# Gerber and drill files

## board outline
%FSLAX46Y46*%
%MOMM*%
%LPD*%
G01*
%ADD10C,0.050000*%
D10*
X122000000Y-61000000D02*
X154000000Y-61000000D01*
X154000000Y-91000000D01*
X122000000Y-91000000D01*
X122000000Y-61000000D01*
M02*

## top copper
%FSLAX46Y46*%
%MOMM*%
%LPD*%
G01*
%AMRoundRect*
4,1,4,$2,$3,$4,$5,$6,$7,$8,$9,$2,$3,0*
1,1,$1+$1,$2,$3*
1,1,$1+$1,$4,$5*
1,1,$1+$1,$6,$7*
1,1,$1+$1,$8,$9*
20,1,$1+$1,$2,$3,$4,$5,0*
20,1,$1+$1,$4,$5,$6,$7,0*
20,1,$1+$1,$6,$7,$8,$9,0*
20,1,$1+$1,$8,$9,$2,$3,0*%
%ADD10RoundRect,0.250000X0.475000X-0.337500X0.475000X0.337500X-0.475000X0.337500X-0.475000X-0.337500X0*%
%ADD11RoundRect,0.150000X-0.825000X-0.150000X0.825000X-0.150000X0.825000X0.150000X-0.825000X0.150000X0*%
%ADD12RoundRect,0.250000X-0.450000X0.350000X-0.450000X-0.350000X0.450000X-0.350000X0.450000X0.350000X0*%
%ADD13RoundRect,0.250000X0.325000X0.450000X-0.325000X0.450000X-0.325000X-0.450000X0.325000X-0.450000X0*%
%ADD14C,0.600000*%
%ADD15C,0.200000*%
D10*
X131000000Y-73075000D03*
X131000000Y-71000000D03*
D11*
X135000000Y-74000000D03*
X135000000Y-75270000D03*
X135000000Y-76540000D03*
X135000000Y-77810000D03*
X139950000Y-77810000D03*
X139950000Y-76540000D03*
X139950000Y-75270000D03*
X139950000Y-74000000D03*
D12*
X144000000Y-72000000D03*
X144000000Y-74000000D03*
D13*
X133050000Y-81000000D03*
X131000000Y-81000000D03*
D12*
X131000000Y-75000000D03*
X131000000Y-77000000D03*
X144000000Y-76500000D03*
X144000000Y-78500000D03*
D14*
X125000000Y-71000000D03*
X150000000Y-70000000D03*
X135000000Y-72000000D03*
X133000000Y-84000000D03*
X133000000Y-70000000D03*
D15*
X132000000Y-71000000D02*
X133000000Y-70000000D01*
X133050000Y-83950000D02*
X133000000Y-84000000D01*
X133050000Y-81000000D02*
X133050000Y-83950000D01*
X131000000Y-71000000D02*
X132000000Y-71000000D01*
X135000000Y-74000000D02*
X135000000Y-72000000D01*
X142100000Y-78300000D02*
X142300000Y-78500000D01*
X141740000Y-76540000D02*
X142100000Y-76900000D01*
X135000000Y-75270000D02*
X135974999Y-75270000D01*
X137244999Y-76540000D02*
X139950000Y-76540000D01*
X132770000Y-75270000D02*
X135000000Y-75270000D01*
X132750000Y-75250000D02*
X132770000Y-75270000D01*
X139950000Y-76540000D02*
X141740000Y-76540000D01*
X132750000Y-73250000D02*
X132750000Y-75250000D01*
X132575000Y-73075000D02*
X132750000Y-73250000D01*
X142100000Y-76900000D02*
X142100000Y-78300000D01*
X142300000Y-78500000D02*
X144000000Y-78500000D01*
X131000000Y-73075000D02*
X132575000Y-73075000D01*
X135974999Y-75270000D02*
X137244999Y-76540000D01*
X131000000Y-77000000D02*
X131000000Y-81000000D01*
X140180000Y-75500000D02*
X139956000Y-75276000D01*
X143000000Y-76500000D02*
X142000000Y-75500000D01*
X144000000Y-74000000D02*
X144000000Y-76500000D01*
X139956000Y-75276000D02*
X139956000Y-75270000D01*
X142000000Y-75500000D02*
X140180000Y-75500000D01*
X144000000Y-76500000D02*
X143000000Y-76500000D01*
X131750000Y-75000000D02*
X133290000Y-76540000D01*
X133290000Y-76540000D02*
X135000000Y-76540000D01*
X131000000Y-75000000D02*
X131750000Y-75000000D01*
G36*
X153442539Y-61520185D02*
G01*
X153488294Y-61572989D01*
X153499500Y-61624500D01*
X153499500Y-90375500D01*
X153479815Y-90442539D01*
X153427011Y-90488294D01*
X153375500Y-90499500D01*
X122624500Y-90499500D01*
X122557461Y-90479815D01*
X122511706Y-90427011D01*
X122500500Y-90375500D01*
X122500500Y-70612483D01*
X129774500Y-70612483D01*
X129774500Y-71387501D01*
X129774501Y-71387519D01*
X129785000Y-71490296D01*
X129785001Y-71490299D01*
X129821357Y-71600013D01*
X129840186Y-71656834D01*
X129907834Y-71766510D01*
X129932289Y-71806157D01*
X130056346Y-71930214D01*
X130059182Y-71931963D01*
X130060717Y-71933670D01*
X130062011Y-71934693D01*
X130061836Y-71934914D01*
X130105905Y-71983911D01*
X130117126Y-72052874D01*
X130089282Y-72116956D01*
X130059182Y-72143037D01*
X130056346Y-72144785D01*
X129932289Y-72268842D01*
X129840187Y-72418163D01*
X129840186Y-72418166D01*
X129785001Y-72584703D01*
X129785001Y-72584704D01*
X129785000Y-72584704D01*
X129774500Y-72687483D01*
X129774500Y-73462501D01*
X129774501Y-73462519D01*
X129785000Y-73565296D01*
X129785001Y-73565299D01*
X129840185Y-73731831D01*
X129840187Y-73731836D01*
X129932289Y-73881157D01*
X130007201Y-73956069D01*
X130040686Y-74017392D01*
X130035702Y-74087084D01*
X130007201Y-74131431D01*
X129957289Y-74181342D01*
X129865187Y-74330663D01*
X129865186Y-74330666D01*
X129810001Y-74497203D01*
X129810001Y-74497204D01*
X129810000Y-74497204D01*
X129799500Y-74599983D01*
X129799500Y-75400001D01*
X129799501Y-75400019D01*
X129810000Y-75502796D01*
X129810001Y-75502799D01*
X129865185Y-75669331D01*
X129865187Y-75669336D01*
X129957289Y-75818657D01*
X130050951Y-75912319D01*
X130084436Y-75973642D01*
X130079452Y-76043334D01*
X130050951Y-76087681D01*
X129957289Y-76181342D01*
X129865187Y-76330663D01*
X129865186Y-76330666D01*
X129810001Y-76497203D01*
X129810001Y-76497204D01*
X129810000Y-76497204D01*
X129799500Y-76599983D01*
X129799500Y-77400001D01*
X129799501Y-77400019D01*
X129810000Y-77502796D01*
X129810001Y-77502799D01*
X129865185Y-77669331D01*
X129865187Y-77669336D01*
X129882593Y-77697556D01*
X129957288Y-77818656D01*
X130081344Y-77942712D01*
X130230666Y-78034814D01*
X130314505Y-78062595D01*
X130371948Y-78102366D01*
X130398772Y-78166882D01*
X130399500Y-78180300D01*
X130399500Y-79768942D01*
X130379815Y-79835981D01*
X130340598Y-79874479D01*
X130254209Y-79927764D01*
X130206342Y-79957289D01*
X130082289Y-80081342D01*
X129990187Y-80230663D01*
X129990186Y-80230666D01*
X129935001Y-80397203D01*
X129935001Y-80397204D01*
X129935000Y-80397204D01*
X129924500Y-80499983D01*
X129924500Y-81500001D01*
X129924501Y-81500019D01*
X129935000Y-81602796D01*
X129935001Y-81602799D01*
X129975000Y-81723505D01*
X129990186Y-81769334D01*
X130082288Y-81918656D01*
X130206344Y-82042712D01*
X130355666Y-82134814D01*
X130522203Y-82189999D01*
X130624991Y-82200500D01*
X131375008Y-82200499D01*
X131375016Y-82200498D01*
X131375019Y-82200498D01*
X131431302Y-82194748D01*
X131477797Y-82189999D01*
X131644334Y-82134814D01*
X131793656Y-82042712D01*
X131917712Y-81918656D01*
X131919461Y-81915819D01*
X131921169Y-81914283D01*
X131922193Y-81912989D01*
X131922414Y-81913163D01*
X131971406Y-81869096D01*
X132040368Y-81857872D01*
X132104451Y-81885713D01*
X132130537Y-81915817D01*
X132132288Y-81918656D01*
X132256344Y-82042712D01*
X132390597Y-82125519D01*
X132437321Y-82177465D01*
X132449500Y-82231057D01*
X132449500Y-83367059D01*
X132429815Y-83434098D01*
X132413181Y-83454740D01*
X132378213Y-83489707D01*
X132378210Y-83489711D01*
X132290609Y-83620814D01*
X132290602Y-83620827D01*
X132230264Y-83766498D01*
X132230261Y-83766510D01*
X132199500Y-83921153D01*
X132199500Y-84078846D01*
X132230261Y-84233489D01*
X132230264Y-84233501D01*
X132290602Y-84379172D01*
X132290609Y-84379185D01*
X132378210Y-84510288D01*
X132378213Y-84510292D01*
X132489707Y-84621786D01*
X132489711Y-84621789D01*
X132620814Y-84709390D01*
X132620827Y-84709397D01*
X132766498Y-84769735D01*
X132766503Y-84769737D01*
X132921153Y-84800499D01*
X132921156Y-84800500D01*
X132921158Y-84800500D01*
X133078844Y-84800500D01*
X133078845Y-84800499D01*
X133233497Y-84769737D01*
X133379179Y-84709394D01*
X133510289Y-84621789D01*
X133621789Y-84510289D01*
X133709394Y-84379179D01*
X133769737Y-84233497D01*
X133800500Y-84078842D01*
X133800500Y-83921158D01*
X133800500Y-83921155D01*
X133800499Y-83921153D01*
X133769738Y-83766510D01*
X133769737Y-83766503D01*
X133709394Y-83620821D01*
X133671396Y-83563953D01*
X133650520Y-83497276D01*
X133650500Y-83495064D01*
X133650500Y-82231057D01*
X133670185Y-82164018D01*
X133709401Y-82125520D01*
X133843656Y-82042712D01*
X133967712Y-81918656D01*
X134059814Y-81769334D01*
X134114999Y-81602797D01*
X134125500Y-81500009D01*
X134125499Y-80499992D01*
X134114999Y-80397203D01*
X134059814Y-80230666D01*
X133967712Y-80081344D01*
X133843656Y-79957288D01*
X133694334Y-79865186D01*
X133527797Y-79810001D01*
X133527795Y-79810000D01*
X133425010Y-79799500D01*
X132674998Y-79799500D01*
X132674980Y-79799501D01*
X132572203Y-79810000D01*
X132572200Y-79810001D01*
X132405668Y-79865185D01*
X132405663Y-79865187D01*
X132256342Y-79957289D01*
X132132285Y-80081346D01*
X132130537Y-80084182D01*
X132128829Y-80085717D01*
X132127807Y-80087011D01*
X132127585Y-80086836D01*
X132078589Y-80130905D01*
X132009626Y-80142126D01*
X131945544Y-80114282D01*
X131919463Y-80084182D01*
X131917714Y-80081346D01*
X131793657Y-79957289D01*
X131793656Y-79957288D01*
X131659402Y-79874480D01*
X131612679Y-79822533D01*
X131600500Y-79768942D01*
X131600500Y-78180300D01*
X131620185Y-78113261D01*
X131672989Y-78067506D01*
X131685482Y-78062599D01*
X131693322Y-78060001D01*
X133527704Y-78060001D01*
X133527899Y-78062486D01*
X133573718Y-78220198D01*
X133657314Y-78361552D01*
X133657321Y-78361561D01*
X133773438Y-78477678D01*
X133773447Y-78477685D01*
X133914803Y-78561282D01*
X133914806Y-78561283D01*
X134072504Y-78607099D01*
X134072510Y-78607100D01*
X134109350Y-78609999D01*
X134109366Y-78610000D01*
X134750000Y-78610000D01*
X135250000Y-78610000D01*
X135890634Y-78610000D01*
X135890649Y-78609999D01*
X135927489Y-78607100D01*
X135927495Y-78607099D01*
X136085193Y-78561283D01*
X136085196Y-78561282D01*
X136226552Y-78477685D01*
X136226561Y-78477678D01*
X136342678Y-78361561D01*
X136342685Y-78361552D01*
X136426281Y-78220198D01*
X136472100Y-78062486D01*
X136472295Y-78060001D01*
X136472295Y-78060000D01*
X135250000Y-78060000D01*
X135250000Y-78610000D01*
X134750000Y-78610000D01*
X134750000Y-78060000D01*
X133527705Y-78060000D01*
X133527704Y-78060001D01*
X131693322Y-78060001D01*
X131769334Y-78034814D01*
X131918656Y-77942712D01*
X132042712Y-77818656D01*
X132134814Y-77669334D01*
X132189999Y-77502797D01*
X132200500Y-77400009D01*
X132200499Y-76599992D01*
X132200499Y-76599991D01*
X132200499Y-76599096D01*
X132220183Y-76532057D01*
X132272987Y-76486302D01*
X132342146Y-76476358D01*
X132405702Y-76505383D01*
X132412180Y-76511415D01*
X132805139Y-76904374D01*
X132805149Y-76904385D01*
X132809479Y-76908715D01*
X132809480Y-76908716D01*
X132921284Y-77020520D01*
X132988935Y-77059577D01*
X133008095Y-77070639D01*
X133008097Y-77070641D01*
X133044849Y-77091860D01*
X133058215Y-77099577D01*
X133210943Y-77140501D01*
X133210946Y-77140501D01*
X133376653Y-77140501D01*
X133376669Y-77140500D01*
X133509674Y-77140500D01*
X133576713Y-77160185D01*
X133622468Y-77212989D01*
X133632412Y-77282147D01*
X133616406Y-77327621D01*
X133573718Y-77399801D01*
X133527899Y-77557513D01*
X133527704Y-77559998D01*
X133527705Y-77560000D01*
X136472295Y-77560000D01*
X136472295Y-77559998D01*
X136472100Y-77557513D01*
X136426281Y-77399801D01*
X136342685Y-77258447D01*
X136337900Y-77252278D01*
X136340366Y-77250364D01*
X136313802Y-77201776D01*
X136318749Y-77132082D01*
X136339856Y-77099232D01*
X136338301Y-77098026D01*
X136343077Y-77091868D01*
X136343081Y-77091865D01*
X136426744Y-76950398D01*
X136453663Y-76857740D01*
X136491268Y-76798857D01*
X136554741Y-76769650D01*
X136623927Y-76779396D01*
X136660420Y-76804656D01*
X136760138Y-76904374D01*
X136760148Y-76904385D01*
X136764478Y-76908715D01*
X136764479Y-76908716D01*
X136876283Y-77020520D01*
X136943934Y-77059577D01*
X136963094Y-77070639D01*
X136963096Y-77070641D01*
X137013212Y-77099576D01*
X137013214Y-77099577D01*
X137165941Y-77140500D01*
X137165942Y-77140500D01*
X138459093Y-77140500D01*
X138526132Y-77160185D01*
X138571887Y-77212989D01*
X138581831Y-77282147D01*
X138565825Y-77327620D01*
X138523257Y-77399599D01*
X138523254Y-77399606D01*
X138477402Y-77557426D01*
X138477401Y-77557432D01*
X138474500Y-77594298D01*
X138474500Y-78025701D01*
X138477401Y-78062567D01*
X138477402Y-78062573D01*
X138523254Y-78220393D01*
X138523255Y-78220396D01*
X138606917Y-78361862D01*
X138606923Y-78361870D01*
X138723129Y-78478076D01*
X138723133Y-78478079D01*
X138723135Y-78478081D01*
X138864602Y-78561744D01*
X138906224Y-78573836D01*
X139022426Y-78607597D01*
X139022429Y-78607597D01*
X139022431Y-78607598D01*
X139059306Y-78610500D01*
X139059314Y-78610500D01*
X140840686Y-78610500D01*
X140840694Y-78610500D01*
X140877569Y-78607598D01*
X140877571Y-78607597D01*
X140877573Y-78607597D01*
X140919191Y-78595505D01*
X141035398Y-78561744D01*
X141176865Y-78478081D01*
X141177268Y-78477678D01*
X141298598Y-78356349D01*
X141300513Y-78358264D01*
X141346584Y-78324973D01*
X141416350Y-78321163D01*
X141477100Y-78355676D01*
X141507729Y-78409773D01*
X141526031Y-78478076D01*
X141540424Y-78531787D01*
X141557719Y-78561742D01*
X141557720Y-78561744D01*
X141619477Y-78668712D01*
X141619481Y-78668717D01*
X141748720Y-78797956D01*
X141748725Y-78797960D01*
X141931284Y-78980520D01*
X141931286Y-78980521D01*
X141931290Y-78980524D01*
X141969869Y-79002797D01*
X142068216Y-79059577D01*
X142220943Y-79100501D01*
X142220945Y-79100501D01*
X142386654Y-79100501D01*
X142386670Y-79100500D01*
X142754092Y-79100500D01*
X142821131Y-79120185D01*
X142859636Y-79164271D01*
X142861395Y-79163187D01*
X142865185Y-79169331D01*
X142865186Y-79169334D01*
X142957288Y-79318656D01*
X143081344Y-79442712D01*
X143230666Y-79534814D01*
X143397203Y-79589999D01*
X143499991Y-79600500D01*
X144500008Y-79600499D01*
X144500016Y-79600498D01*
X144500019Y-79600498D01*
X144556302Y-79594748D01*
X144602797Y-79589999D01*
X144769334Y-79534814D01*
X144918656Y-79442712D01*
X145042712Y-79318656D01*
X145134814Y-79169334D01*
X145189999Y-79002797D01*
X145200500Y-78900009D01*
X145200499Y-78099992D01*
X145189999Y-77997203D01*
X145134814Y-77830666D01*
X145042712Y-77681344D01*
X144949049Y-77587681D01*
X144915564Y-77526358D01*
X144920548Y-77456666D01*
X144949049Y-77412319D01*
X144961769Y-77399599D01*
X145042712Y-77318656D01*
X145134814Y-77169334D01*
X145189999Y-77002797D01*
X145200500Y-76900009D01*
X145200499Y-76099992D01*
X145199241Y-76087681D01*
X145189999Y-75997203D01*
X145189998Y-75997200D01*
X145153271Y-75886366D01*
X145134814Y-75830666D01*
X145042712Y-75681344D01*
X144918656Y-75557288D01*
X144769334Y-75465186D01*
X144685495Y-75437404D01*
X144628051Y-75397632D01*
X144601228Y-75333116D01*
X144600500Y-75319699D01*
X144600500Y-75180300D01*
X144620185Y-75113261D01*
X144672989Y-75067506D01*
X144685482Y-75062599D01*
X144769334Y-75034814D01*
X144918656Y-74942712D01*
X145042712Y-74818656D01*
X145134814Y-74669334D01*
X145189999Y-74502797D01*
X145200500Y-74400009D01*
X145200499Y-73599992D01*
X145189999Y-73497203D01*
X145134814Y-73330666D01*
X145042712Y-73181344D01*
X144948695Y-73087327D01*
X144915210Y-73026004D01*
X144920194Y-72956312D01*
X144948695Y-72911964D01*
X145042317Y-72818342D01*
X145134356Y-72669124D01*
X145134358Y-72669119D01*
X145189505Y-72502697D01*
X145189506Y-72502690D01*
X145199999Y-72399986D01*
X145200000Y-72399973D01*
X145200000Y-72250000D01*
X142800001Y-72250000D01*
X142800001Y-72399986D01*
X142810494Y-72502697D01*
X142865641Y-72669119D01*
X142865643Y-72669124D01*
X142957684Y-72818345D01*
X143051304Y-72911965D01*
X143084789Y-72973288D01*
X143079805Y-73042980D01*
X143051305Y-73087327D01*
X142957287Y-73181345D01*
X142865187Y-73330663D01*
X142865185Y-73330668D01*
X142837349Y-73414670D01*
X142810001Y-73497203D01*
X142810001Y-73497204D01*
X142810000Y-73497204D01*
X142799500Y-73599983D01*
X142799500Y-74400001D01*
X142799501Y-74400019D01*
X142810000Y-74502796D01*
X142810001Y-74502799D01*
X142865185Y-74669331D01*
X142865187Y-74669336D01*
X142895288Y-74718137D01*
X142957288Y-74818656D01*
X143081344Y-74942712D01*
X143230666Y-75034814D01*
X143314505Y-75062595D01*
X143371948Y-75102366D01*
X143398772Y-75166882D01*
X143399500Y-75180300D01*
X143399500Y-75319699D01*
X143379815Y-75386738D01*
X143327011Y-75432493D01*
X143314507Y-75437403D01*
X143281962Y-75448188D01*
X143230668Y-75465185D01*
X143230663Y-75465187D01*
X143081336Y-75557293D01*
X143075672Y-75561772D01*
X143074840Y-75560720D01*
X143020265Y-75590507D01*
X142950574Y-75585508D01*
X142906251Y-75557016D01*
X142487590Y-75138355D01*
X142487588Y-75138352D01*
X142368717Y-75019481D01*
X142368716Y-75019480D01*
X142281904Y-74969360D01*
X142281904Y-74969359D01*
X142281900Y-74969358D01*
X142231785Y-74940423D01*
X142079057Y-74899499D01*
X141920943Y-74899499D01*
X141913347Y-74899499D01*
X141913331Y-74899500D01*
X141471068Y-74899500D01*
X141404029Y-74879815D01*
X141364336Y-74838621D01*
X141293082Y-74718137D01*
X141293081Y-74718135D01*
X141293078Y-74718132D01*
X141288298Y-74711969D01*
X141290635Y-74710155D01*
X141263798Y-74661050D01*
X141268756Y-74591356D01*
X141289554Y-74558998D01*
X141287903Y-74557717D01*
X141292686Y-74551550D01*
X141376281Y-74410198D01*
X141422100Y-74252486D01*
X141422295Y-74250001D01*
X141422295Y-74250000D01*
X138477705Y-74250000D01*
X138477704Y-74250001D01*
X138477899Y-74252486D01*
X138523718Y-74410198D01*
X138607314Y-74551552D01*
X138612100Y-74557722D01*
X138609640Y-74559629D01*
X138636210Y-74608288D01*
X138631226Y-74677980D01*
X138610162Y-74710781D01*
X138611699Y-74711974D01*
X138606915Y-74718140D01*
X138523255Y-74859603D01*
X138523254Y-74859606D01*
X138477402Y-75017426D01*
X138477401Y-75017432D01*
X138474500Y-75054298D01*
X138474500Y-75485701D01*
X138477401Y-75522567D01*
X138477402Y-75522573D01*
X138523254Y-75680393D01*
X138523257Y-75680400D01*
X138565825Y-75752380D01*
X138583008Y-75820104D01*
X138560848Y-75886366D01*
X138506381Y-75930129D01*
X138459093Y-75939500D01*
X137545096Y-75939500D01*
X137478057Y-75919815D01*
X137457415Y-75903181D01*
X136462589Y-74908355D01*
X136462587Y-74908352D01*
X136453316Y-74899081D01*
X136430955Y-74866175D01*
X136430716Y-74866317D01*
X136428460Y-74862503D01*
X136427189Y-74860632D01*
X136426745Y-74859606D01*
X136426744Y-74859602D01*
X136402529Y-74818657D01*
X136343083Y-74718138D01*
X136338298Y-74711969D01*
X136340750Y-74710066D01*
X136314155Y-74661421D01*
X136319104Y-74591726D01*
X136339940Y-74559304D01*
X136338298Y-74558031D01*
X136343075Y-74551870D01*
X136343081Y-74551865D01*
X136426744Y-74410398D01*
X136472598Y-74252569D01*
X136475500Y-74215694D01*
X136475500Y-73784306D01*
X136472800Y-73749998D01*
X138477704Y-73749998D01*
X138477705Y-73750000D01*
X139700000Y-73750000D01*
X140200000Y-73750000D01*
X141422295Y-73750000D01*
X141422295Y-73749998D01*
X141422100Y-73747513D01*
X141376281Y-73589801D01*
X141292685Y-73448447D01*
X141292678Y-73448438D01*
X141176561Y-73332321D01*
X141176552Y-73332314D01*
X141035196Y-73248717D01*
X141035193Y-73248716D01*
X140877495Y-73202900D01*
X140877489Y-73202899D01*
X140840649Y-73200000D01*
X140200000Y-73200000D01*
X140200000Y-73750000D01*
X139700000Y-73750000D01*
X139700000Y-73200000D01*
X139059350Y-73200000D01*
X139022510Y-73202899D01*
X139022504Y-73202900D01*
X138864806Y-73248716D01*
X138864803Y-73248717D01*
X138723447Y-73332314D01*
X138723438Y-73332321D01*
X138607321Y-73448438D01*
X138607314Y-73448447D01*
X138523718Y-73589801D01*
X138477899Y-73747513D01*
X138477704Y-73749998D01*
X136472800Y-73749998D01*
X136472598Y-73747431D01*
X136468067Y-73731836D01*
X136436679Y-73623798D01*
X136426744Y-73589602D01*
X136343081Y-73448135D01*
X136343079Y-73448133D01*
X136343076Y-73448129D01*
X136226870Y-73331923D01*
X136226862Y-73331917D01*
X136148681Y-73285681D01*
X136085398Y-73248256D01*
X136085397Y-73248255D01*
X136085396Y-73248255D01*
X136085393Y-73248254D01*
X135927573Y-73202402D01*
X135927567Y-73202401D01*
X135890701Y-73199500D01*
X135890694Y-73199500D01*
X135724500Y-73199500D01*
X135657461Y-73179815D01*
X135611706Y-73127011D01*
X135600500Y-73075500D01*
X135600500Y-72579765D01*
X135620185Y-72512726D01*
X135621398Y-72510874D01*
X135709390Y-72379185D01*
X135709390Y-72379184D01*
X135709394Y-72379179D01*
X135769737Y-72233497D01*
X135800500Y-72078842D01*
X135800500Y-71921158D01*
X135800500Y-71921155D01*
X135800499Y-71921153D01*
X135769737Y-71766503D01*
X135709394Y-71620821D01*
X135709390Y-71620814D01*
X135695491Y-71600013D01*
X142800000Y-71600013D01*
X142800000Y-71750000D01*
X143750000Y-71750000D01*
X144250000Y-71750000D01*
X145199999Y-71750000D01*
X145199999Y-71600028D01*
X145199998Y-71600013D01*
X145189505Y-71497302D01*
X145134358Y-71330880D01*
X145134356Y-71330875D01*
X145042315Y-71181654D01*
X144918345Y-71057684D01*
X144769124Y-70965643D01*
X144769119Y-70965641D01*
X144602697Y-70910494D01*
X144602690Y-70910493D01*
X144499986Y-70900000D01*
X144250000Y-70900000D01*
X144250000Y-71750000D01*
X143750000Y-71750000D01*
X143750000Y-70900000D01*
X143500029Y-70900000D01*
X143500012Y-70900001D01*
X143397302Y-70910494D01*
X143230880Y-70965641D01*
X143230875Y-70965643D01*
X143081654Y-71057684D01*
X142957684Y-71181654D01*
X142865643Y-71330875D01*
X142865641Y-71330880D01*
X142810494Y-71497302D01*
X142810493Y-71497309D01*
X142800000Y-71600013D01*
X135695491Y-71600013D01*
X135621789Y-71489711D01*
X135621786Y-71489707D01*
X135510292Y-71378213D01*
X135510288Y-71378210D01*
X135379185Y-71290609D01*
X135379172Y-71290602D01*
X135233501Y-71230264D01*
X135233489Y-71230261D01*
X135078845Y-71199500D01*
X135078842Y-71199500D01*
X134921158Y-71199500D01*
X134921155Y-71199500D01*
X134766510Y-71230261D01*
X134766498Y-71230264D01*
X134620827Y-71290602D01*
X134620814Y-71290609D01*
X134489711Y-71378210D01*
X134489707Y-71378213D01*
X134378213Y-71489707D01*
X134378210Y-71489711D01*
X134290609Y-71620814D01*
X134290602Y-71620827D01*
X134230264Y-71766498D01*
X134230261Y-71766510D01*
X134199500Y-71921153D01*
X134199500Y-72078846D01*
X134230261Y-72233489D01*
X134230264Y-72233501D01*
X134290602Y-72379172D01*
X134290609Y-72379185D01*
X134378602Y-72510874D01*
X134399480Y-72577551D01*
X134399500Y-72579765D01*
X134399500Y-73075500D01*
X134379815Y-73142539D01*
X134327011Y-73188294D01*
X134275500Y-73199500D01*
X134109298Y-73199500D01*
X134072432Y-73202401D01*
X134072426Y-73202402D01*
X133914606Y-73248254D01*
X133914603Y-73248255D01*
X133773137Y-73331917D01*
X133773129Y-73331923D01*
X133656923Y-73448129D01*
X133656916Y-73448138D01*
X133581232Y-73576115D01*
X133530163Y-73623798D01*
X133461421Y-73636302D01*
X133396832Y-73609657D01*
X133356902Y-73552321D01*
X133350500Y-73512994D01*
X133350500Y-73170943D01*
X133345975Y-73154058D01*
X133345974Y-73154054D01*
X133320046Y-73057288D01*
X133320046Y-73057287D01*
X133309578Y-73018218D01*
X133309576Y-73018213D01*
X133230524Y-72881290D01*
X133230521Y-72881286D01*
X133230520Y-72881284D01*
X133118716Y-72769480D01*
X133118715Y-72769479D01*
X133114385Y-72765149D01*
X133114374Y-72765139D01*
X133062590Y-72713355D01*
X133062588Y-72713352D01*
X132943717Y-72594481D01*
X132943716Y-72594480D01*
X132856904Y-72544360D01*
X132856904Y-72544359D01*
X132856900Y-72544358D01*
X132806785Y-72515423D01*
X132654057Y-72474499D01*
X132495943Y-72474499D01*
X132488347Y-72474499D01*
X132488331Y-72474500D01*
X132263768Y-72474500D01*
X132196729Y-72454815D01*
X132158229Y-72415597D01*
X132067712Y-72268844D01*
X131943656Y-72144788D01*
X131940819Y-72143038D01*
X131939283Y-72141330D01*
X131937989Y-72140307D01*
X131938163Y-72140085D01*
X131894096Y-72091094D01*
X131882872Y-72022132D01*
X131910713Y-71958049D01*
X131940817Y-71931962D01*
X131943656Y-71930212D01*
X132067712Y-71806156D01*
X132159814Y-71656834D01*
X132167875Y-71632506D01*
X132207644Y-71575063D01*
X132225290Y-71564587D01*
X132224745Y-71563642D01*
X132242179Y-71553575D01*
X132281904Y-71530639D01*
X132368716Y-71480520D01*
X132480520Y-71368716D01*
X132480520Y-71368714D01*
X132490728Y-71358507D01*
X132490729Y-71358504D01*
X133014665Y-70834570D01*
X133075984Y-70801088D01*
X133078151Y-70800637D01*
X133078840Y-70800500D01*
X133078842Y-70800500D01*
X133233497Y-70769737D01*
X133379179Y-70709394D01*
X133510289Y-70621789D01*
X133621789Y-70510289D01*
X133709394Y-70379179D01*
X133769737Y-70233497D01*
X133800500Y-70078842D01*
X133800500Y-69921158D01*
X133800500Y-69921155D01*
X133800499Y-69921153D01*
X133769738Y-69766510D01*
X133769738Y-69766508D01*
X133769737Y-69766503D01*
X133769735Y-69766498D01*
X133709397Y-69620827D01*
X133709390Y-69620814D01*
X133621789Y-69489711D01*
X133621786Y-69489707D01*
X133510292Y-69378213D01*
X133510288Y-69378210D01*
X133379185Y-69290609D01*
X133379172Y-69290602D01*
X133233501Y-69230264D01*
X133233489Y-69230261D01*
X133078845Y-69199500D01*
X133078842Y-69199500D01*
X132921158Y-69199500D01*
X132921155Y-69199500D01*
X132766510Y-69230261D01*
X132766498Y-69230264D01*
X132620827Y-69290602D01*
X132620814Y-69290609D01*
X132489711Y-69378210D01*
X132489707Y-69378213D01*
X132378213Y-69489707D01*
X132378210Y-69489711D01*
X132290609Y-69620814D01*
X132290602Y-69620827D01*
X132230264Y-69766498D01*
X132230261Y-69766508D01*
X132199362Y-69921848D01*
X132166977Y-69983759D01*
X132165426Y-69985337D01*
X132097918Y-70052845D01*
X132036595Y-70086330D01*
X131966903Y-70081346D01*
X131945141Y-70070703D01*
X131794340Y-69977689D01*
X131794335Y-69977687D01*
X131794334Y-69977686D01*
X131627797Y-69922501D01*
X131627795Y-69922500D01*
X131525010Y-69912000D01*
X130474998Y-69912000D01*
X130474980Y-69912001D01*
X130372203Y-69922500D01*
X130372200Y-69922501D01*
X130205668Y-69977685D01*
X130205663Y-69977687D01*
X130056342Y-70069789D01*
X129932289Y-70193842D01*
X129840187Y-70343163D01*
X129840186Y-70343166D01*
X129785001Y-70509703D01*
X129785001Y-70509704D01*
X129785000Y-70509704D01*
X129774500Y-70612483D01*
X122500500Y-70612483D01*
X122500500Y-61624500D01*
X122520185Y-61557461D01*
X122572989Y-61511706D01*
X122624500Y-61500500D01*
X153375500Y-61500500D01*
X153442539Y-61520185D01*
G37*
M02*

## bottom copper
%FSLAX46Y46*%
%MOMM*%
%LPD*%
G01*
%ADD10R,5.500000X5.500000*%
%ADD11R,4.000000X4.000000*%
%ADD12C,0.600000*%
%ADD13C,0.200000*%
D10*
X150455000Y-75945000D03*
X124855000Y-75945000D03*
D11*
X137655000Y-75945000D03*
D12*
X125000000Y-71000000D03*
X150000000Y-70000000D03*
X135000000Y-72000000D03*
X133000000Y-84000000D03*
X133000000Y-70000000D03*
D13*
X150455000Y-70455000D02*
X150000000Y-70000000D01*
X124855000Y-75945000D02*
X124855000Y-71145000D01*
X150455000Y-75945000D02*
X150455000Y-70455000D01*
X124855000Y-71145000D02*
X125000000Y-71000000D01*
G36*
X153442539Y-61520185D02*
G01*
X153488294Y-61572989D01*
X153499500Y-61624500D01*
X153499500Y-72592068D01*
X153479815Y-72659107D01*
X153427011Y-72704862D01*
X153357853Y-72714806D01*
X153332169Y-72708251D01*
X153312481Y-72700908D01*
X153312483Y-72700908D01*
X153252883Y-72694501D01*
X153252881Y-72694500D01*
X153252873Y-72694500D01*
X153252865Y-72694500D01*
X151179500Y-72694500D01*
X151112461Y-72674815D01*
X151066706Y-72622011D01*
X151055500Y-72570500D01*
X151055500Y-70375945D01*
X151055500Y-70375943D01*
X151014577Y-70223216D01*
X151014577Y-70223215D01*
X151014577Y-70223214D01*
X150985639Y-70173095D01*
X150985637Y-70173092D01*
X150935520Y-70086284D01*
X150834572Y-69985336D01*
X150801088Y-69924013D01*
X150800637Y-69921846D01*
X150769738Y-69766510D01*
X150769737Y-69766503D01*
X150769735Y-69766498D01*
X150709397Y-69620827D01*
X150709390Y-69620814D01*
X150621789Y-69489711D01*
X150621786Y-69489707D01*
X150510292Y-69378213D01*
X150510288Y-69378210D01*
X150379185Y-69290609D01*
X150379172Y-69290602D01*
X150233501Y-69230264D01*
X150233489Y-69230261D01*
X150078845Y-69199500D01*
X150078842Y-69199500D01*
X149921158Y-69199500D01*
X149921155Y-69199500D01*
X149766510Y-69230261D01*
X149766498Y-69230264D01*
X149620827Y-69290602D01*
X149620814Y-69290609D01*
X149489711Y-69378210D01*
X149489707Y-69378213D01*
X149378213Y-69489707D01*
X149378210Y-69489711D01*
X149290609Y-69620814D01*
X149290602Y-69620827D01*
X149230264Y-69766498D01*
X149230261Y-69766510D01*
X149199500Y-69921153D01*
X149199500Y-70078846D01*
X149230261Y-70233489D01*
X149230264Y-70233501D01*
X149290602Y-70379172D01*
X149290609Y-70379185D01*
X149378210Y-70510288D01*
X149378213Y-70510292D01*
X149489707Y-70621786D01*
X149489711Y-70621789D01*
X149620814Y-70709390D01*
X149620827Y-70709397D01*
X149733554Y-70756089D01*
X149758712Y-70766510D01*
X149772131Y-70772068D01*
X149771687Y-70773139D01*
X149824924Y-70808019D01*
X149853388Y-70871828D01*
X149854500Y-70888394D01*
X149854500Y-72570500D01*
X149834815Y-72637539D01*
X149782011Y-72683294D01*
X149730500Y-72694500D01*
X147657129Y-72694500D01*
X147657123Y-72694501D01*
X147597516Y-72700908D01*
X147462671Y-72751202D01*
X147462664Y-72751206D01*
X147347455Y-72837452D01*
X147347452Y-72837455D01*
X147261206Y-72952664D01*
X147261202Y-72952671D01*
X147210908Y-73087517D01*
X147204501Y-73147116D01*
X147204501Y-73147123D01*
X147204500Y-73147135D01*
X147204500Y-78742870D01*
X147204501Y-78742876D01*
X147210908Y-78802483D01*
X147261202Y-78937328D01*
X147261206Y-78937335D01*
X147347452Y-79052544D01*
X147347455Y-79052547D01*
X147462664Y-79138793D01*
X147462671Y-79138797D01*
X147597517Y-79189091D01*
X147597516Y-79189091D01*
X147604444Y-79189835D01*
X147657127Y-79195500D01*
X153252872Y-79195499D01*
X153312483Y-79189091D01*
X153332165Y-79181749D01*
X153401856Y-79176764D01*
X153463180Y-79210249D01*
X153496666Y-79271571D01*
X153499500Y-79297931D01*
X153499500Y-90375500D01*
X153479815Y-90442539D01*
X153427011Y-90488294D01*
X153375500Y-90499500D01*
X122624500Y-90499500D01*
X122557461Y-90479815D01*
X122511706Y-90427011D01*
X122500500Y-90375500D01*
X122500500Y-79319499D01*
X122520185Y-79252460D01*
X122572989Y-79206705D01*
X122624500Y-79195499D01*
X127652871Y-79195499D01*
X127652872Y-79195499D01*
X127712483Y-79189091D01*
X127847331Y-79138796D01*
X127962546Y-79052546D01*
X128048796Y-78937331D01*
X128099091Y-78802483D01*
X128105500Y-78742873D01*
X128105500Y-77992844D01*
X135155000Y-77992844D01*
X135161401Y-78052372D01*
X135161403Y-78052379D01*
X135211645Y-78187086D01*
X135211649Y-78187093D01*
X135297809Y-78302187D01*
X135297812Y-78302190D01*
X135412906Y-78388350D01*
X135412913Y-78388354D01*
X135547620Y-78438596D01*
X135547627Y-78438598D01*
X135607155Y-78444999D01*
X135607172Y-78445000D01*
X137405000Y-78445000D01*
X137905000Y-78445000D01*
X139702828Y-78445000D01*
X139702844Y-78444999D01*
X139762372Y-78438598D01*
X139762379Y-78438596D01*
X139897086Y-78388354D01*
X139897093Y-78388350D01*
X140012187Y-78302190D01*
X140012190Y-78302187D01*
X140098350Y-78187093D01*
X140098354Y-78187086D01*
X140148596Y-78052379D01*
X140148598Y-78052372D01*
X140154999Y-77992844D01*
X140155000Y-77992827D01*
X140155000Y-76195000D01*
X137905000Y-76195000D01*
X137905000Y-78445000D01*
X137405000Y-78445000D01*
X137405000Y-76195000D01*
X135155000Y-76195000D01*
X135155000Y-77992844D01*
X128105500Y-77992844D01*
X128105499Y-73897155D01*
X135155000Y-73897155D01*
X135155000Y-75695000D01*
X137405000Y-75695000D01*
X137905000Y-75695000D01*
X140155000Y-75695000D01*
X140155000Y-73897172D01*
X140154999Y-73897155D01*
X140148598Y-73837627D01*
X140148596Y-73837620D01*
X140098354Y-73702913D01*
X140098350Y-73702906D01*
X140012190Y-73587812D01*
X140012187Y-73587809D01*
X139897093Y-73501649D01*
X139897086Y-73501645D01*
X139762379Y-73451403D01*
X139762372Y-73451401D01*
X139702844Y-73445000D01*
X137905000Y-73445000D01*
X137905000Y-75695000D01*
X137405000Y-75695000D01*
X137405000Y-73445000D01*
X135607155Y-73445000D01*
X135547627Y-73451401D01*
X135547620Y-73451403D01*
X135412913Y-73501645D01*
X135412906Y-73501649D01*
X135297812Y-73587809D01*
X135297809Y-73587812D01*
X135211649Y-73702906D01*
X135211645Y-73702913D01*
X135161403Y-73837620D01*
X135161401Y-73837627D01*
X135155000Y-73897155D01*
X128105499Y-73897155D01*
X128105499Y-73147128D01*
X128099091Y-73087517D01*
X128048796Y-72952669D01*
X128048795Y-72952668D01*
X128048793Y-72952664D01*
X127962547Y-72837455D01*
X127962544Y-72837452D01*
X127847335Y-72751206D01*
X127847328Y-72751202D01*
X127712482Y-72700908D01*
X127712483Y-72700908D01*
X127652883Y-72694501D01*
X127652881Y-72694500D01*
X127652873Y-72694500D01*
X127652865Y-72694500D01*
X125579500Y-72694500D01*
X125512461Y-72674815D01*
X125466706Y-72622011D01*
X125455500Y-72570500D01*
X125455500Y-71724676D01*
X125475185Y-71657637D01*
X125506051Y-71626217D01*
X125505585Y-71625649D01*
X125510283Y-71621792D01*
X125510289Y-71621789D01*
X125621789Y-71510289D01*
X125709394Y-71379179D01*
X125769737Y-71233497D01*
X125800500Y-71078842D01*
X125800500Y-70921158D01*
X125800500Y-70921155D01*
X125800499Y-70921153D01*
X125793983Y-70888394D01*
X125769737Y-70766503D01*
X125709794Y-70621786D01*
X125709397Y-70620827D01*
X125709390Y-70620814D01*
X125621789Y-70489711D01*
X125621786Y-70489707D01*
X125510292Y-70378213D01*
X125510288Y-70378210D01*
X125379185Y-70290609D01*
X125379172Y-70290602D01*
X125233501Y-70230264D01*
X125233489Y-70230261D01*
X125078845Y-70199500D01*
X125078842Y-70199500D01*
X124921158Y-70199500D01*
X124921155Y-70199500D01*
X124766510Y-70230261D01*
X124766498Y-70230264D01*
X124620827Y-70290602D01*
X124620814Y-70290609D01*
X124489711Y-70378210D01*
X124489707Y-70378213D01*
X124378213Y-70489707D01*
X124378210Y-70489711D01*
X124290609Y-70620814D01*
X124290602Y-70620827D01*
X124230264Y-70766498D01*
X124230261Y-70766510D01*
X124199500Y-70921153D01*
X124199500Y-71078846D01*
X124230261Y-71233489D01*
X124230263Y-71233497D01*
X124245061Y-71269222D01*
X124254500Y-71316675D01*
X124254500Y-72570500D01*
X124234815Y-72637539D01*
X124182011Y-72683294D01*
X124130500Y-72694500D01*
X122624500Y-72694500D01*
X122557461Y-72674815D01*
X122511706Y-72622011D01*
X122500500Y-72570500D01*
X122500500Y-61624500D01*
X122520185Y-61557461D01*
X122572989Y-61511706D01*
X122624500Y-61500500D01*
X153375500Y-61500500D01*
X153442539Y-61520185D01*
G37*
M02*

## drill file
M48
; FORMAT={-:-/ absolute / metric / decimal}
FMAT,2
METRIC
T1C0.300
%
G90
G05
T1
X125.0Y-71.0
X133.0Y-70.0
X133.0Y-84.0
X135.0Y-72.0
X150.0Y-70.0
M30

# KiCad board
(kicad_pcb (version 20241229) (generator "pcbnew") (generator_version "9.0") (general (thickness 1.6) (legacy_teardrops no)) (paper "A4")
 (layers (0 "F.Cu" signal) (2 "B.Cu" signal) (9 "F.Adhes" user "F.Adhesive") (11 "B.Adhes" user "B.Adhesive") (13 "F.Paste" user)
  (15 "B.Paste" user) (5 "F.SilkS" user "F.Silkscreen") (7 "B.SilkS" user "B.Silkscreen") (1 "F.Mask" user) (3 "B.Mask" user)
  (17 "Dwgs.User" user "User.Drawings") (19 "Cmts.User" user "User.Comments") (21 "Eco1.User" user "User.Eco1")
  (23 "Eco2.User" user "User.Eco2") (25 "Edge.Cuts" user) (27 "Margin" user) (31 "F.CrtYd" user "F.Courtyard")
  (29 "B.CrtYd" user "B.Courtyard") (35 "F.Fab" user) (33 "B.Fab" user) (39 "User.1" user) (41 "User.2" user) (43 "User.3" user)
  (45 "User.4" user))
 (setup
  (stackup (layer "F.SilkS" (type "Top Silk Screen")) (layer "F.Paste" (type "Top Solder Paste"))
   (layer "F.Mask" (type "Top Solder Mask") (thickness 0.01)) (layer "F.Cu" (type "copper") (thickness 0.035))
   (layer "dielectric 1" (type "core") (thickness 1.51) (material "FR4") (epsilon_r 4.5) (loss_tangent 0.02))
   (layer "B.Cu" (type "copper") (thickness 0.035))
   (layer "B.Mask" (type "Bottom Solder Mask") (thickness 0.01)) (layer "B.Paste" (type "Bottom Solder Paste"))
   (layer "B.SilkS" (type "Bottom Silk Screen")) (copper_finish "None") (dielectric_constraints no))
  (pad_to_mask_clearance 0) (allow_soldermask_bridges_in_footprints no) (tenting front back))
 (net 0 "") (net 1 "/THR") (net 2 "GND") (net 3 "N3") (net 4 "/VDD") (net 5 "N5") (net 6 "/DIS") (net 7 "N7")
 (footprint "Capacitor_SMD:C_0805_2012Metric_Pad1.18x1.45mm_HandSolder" (layer "F.Cu") (at 131 72.0375 90)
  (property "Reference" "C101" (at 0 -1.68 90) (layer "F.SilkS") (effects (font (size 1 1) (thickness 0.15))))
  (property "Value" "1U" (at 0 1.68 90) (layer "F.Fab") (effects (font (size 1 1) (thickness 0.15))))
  (pad "1" smd roundrect (at -1.0375 0 90) (size 1.175 1.45) (layers "F.Cu" "F.Mask" "F.Paste") (roundrect_rratio 0.212766) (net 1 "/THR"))
  (pad "2" smd roundrect (at 1.0375 0 90) (size 1.175 1.45) (layers "F.Cu" "F.Mask" "F.Paste") (roundrect_rratio 0.212766) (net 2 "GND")))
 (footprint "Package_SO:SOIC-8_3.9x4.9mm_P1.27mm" (layer "F.Cu") (at 137.475 75.905)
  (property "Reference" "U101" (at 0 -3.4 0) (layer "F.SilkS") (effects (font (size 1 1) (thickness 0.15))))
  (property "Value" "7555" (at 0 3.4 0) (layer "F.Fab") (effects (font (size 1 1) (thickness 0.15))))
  (pad "1" smd roundrect (at -2.475 -1.905) (size 1.95 0.6) (layers "F.Cu" "F.Mask" "F.Paste") (roundrect_rratio 0.25) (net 2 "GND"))
  (pad "2" smd roundrect (at -2.475 -0.635) (size 1.95 0.6) (layers "F.Cu" "F.Mask" "F.Paste") (roundrect_rratio 0.25) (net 1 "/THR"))
  (pad "3" smd roundrect (at -2.475 0.635) (size 1.95 0.6) (layers "F.Cu" "F.Mask" "F.Paste") (roundrect_rratio 0.25) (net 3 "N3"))
  (pad "4" smd roundrect (at -2.475 1.905) (size 1.95 0.6) (layers "F.Cu" "F.Mask" "F.Paste") (roundrect_rratio 0.25) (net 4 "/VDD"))
  (pad "5" smd roundrect (at 2.475 1.905) (size 1.95 0.6) (layers "F.Cu" "F.Mask" "F.Paste") (roundrect_rratio 0.25) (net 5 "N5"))
  (pad "6" smd roundrect (at 2.475 0.635) (size 1.95 0.6) (layers "F.Cu" "F.Mask" "F.Paste") (roundrect_rratio 0.25) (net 1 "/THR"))
  (pad "7" smd roundrect (at 2.475 -0.635) (size 1.95 0.6) (layers "F.Cu" "F.Mask" "F.Paste") (roundrect_rratio 0.25) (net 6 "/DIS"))
  (pad "8" smd roundrect (at 2.475 -1.905) (size 1.95 0.6) (layers "F.Cu" "F.Mask" "F.Paste") (roundrect_rratio 0.25) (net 4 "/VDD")))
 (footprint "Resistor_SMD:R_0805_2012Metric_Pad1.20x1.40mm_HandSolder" (layer "F.Cu") (at 144 73 -90)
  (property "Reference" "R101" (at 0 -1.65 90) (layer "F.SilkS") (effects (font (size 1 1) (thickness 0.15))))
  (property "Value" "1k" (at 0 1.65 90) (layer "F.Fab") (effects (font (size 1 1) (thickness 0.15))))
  (pad "1" smd roundrect (at -1 0 270) (size 1.2 1.4) (layers "F.Cu" "F.Mask" "F.Paste") (roundrect_rratio 0.208333) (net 4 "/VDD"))
  (pad "2" smd roundrect (at 1 0 270) (size 1.2 1.4) (layers "F.Cu" "F.Mask" "F.Paste") (roundrect_rratio 0.208333) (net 6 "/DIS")))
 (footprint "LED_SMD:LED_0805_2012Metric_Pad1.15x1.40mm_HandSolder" (layer "F.Cu") (at 132.025 81 180)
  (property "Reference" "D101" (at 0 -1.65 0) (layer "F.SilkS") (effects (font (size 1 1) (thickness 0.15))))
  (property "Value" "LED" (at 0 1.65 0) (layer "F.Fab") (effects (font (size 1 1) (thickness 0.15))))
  (pad "1" smd roundrect (at -1.025 0 180) (size 1.15 1.4) (layers "F.Cu" "F.Mask" "F.Paste") (roundrect_rratio 0.217391) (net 2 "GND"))
  (pad "2" smd roundrect (at 1.025 0 180) (size 1.15 1.4) (layers "F.Cu" "F.Mask" "F.Paste") (roundrect_rratio 0.217391) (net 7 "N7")))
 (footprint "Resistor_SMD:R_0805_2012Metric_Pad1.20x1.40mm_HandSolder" (layer "F.Cu") (at 131 76 -90)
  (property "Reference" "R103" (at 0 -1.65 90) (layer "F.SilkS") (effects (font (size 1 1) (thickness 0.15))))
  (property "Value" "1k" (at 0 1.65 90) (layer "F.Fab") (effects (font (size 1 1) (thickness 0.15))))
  (pad "1" smd roundrect (at -1 0 270) (size 1.2 1.4) (layers "F.Cu" "F.Mask" "F.Paste") (roundrect_rratio 0.208333) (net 3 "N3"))
  (pad "2" smd roundrect (at 1 0 270) (size 1.2 1.4) (layers "F.Cu" "F.Mask" "F.Paste") (roundrect_rratio 0.208333) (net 7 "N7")))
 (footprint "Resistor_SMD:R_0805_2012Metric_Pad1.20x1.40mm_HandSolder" (layer "F.Cu") (at 144 77.5 -90)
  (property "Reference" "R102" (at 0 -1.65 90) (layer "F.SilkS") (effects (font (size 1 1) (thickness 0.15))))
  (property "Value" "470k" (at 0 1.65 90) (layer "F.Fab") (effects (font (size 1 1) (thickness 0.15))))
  (pad "1" smd roundrect (at -1 0 270) (size 1.2 1.4) (layers "F.Cu" "F.Mask" "F.Paste") (roundrect_rratio 0.208333) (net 6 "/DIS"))
  (pad "2" smd roundrect (at 1 0 270) (size 1.2 1.4) (layers "F.Cu" "F.Mask" "F.Paste") (roundrect_rratio 0.208333) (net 1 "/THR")))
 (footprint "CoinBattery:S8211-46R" (layer "B.Cu") (at 137.655 75.945 180)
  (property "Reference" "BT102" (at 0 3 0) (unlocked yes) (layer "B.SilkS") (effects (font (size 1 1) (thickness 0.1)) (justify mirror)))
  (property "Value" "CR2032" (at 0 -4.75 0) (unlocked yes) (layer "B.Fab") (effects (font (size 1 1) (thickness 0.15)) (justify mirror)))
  (pad "1" smd rect (at -12.8 0 180) (size 5.5 5.5) (layers "B.Cu" "B.Mask" "B.Paste") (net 4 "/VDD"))
  (pad "1" smd rect (at 12.8 0 180) (size 5.5 5.5) (layers "B.Cu" "B.Mask" "B.Paste") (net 4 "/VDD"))
  (pad "2" smd rect (at 0 0 180) (size 4 4) (layers "B.Cu" "B.Mask" "B.Paste") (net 2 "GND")))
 (gr_rect (start 122 61) (end 154 91) (stroke (width 0.05) (type default)) (fill no) (layer "Edge.Cuts"))
 (via (at 125 71) (size 0.6) (drill 0.3) (layers "F.Cu" "B.Cu") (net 4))
 (via (at 150 70) (size 0.6) (drill 0.3) (layers "F.Cu" "B.Cu") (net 4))
 (segment (start 150.455 70.455) (end 150 70) (width 0.2) (layer "B.Cu") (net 4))
 (segment (start 124.855 75.945) (end 124.855 71.145) (width 0.2) (layer "B.Cu") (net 4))
 (segment (start 150.455 75.945) (end 150.455 70.455) (width 0.2) (layer "B.Cu") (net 4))
 (segment (start 124.855 71.145) (end 125 71) (width 0.2) (layer "B.Cu") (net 4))
 (segment (start 132 71) (end 133 70) (width 0.2) (layer "F.Cu") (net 2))
 (segment (start 133.05 83.95) (end 133 84) (width 0.2) (layer "F.Cu") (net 2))
 (segment (start 133.05 81) (end 133.05 83.95) (width 0.2) (layer "F.Cu") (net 2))
 (segment (start 131 71) (end 132 71) (width 0.2) (layer "F.Cu") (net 2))
 (segment (start 135 74) (end 135 72) (width 0.2) (layer "F.Cu") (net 2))
 (via (at 135 72) (size 0.6) (drill 0.3) (layers "F.Cu" "B.Cu") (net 2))
 (via (at 133 84) (size 0.6) (drill 0.3) (layers "F.Cu" "B.Cu") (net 2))
 (via (at 133 70) (size 0.6) (drill 0.3) (layers "F.Cu" "B.Cu") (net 2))
 (segment (start 142.1 78.3) (end 142.3 78.5) (width 0.2) (layer "F.Cu") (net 1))
 (segment (start 141.74 76.54) (end 142.1 76.9) (width 0.2) (layer "F.Cu") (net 1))
 (segment (start 135 75.27) (end 135.974999 75.27) (width 0.2) (layer "F.Cu") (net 1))
 (segment (start 137.244999 76.54) (end 139.95 76.54) (width 0.2) (layer "F.Cu") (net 1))
 (segment (start 132.77 75.27) (end 135 75.27) (width 0.2) (layer "F.Cu") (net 1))
 (segment (start 132.75 75.25) (end 132.77 75.27) (width 0.2) (layer "F.Cu") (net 1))
 (segment (start 139.95 76.54) (end 141.74 76.54) (width 0.2) (layer "F.Cu") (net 1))
 (segment (start 132.75 73.25) (end 132.75 75.25) (width 0.2) (layer "F.Cu") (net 1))
 (segment (start 132.575 73.075) (end 132.75 73.25) (width 0.2) (layer "F.Cu") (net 1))
 (segment (start 142.1 76.9) (end 142.1 78.3) (width 0.2) (layer "F.Cu") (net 1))
 (segment (start 142.3 78.5) (end 144 78.5) (width 0.2) (layer "F.Cu") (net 1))
 (segment (start 131 73.075) (end 132.575 73.075) (width 0.2) (layer "F.Cu") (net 1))
 (segment (start 135.974999 75.27) (end 137.244999 76.54) (width 0.2) (layer "F.Cu") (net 1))
 (segment (start 131 77) (end 131 81) (width 0.2) (layer "F.Cu") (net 7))
 (segment (start 140.18 75.5) (end 139.956 75.276) (width 0.2) (layer "F.Cu") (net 6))
 (segment (start 143 76.5) (end 142 75.5) (width 0.2) (layer "F.Cu") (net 6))
 (segment (start 144 74) (end 144 76.5) (width 0.2) (layer "F.Cu") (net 6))
 (segment (start 139.956 75.276) (end 139.956 75.27) (width 0.2) (layer "F.Cu") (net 6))
 (segment (start 142 75.5) (end 140.18 75.5) (width 0.2) (layer "F.Cu") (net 6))
 (segment (start 144 76.5) (end 143 76.5) (width 0.2) (layer "F.Cu") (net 6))
 (segment (start 131.75 75) (end 133.29 76.54) (width 0.2) (layer "F.Cu") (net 3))
 (segment (start 133.29 76.54) (end 135 76.54) (width 0.2) (layer "F.Cu") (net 3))
 (segment (start 131 75) (end 131.75 75) (width 0.2) (layer "F.Cu") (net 3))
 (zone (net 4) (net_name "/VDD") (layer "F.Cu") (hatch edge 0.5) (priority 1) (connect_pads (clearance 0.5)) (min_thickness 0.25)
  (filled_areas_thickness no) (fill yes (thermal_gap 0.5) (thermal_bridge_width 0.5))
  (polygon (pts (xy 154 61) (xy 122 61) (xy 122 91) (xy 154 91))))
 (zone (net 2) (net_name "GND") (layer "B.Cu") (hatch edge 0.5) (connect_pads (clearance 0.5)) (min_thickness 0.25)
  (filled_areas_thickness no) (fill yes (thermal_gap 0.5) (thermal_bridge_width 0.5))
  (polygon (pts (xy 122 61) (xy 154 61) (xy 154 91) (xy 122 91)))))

